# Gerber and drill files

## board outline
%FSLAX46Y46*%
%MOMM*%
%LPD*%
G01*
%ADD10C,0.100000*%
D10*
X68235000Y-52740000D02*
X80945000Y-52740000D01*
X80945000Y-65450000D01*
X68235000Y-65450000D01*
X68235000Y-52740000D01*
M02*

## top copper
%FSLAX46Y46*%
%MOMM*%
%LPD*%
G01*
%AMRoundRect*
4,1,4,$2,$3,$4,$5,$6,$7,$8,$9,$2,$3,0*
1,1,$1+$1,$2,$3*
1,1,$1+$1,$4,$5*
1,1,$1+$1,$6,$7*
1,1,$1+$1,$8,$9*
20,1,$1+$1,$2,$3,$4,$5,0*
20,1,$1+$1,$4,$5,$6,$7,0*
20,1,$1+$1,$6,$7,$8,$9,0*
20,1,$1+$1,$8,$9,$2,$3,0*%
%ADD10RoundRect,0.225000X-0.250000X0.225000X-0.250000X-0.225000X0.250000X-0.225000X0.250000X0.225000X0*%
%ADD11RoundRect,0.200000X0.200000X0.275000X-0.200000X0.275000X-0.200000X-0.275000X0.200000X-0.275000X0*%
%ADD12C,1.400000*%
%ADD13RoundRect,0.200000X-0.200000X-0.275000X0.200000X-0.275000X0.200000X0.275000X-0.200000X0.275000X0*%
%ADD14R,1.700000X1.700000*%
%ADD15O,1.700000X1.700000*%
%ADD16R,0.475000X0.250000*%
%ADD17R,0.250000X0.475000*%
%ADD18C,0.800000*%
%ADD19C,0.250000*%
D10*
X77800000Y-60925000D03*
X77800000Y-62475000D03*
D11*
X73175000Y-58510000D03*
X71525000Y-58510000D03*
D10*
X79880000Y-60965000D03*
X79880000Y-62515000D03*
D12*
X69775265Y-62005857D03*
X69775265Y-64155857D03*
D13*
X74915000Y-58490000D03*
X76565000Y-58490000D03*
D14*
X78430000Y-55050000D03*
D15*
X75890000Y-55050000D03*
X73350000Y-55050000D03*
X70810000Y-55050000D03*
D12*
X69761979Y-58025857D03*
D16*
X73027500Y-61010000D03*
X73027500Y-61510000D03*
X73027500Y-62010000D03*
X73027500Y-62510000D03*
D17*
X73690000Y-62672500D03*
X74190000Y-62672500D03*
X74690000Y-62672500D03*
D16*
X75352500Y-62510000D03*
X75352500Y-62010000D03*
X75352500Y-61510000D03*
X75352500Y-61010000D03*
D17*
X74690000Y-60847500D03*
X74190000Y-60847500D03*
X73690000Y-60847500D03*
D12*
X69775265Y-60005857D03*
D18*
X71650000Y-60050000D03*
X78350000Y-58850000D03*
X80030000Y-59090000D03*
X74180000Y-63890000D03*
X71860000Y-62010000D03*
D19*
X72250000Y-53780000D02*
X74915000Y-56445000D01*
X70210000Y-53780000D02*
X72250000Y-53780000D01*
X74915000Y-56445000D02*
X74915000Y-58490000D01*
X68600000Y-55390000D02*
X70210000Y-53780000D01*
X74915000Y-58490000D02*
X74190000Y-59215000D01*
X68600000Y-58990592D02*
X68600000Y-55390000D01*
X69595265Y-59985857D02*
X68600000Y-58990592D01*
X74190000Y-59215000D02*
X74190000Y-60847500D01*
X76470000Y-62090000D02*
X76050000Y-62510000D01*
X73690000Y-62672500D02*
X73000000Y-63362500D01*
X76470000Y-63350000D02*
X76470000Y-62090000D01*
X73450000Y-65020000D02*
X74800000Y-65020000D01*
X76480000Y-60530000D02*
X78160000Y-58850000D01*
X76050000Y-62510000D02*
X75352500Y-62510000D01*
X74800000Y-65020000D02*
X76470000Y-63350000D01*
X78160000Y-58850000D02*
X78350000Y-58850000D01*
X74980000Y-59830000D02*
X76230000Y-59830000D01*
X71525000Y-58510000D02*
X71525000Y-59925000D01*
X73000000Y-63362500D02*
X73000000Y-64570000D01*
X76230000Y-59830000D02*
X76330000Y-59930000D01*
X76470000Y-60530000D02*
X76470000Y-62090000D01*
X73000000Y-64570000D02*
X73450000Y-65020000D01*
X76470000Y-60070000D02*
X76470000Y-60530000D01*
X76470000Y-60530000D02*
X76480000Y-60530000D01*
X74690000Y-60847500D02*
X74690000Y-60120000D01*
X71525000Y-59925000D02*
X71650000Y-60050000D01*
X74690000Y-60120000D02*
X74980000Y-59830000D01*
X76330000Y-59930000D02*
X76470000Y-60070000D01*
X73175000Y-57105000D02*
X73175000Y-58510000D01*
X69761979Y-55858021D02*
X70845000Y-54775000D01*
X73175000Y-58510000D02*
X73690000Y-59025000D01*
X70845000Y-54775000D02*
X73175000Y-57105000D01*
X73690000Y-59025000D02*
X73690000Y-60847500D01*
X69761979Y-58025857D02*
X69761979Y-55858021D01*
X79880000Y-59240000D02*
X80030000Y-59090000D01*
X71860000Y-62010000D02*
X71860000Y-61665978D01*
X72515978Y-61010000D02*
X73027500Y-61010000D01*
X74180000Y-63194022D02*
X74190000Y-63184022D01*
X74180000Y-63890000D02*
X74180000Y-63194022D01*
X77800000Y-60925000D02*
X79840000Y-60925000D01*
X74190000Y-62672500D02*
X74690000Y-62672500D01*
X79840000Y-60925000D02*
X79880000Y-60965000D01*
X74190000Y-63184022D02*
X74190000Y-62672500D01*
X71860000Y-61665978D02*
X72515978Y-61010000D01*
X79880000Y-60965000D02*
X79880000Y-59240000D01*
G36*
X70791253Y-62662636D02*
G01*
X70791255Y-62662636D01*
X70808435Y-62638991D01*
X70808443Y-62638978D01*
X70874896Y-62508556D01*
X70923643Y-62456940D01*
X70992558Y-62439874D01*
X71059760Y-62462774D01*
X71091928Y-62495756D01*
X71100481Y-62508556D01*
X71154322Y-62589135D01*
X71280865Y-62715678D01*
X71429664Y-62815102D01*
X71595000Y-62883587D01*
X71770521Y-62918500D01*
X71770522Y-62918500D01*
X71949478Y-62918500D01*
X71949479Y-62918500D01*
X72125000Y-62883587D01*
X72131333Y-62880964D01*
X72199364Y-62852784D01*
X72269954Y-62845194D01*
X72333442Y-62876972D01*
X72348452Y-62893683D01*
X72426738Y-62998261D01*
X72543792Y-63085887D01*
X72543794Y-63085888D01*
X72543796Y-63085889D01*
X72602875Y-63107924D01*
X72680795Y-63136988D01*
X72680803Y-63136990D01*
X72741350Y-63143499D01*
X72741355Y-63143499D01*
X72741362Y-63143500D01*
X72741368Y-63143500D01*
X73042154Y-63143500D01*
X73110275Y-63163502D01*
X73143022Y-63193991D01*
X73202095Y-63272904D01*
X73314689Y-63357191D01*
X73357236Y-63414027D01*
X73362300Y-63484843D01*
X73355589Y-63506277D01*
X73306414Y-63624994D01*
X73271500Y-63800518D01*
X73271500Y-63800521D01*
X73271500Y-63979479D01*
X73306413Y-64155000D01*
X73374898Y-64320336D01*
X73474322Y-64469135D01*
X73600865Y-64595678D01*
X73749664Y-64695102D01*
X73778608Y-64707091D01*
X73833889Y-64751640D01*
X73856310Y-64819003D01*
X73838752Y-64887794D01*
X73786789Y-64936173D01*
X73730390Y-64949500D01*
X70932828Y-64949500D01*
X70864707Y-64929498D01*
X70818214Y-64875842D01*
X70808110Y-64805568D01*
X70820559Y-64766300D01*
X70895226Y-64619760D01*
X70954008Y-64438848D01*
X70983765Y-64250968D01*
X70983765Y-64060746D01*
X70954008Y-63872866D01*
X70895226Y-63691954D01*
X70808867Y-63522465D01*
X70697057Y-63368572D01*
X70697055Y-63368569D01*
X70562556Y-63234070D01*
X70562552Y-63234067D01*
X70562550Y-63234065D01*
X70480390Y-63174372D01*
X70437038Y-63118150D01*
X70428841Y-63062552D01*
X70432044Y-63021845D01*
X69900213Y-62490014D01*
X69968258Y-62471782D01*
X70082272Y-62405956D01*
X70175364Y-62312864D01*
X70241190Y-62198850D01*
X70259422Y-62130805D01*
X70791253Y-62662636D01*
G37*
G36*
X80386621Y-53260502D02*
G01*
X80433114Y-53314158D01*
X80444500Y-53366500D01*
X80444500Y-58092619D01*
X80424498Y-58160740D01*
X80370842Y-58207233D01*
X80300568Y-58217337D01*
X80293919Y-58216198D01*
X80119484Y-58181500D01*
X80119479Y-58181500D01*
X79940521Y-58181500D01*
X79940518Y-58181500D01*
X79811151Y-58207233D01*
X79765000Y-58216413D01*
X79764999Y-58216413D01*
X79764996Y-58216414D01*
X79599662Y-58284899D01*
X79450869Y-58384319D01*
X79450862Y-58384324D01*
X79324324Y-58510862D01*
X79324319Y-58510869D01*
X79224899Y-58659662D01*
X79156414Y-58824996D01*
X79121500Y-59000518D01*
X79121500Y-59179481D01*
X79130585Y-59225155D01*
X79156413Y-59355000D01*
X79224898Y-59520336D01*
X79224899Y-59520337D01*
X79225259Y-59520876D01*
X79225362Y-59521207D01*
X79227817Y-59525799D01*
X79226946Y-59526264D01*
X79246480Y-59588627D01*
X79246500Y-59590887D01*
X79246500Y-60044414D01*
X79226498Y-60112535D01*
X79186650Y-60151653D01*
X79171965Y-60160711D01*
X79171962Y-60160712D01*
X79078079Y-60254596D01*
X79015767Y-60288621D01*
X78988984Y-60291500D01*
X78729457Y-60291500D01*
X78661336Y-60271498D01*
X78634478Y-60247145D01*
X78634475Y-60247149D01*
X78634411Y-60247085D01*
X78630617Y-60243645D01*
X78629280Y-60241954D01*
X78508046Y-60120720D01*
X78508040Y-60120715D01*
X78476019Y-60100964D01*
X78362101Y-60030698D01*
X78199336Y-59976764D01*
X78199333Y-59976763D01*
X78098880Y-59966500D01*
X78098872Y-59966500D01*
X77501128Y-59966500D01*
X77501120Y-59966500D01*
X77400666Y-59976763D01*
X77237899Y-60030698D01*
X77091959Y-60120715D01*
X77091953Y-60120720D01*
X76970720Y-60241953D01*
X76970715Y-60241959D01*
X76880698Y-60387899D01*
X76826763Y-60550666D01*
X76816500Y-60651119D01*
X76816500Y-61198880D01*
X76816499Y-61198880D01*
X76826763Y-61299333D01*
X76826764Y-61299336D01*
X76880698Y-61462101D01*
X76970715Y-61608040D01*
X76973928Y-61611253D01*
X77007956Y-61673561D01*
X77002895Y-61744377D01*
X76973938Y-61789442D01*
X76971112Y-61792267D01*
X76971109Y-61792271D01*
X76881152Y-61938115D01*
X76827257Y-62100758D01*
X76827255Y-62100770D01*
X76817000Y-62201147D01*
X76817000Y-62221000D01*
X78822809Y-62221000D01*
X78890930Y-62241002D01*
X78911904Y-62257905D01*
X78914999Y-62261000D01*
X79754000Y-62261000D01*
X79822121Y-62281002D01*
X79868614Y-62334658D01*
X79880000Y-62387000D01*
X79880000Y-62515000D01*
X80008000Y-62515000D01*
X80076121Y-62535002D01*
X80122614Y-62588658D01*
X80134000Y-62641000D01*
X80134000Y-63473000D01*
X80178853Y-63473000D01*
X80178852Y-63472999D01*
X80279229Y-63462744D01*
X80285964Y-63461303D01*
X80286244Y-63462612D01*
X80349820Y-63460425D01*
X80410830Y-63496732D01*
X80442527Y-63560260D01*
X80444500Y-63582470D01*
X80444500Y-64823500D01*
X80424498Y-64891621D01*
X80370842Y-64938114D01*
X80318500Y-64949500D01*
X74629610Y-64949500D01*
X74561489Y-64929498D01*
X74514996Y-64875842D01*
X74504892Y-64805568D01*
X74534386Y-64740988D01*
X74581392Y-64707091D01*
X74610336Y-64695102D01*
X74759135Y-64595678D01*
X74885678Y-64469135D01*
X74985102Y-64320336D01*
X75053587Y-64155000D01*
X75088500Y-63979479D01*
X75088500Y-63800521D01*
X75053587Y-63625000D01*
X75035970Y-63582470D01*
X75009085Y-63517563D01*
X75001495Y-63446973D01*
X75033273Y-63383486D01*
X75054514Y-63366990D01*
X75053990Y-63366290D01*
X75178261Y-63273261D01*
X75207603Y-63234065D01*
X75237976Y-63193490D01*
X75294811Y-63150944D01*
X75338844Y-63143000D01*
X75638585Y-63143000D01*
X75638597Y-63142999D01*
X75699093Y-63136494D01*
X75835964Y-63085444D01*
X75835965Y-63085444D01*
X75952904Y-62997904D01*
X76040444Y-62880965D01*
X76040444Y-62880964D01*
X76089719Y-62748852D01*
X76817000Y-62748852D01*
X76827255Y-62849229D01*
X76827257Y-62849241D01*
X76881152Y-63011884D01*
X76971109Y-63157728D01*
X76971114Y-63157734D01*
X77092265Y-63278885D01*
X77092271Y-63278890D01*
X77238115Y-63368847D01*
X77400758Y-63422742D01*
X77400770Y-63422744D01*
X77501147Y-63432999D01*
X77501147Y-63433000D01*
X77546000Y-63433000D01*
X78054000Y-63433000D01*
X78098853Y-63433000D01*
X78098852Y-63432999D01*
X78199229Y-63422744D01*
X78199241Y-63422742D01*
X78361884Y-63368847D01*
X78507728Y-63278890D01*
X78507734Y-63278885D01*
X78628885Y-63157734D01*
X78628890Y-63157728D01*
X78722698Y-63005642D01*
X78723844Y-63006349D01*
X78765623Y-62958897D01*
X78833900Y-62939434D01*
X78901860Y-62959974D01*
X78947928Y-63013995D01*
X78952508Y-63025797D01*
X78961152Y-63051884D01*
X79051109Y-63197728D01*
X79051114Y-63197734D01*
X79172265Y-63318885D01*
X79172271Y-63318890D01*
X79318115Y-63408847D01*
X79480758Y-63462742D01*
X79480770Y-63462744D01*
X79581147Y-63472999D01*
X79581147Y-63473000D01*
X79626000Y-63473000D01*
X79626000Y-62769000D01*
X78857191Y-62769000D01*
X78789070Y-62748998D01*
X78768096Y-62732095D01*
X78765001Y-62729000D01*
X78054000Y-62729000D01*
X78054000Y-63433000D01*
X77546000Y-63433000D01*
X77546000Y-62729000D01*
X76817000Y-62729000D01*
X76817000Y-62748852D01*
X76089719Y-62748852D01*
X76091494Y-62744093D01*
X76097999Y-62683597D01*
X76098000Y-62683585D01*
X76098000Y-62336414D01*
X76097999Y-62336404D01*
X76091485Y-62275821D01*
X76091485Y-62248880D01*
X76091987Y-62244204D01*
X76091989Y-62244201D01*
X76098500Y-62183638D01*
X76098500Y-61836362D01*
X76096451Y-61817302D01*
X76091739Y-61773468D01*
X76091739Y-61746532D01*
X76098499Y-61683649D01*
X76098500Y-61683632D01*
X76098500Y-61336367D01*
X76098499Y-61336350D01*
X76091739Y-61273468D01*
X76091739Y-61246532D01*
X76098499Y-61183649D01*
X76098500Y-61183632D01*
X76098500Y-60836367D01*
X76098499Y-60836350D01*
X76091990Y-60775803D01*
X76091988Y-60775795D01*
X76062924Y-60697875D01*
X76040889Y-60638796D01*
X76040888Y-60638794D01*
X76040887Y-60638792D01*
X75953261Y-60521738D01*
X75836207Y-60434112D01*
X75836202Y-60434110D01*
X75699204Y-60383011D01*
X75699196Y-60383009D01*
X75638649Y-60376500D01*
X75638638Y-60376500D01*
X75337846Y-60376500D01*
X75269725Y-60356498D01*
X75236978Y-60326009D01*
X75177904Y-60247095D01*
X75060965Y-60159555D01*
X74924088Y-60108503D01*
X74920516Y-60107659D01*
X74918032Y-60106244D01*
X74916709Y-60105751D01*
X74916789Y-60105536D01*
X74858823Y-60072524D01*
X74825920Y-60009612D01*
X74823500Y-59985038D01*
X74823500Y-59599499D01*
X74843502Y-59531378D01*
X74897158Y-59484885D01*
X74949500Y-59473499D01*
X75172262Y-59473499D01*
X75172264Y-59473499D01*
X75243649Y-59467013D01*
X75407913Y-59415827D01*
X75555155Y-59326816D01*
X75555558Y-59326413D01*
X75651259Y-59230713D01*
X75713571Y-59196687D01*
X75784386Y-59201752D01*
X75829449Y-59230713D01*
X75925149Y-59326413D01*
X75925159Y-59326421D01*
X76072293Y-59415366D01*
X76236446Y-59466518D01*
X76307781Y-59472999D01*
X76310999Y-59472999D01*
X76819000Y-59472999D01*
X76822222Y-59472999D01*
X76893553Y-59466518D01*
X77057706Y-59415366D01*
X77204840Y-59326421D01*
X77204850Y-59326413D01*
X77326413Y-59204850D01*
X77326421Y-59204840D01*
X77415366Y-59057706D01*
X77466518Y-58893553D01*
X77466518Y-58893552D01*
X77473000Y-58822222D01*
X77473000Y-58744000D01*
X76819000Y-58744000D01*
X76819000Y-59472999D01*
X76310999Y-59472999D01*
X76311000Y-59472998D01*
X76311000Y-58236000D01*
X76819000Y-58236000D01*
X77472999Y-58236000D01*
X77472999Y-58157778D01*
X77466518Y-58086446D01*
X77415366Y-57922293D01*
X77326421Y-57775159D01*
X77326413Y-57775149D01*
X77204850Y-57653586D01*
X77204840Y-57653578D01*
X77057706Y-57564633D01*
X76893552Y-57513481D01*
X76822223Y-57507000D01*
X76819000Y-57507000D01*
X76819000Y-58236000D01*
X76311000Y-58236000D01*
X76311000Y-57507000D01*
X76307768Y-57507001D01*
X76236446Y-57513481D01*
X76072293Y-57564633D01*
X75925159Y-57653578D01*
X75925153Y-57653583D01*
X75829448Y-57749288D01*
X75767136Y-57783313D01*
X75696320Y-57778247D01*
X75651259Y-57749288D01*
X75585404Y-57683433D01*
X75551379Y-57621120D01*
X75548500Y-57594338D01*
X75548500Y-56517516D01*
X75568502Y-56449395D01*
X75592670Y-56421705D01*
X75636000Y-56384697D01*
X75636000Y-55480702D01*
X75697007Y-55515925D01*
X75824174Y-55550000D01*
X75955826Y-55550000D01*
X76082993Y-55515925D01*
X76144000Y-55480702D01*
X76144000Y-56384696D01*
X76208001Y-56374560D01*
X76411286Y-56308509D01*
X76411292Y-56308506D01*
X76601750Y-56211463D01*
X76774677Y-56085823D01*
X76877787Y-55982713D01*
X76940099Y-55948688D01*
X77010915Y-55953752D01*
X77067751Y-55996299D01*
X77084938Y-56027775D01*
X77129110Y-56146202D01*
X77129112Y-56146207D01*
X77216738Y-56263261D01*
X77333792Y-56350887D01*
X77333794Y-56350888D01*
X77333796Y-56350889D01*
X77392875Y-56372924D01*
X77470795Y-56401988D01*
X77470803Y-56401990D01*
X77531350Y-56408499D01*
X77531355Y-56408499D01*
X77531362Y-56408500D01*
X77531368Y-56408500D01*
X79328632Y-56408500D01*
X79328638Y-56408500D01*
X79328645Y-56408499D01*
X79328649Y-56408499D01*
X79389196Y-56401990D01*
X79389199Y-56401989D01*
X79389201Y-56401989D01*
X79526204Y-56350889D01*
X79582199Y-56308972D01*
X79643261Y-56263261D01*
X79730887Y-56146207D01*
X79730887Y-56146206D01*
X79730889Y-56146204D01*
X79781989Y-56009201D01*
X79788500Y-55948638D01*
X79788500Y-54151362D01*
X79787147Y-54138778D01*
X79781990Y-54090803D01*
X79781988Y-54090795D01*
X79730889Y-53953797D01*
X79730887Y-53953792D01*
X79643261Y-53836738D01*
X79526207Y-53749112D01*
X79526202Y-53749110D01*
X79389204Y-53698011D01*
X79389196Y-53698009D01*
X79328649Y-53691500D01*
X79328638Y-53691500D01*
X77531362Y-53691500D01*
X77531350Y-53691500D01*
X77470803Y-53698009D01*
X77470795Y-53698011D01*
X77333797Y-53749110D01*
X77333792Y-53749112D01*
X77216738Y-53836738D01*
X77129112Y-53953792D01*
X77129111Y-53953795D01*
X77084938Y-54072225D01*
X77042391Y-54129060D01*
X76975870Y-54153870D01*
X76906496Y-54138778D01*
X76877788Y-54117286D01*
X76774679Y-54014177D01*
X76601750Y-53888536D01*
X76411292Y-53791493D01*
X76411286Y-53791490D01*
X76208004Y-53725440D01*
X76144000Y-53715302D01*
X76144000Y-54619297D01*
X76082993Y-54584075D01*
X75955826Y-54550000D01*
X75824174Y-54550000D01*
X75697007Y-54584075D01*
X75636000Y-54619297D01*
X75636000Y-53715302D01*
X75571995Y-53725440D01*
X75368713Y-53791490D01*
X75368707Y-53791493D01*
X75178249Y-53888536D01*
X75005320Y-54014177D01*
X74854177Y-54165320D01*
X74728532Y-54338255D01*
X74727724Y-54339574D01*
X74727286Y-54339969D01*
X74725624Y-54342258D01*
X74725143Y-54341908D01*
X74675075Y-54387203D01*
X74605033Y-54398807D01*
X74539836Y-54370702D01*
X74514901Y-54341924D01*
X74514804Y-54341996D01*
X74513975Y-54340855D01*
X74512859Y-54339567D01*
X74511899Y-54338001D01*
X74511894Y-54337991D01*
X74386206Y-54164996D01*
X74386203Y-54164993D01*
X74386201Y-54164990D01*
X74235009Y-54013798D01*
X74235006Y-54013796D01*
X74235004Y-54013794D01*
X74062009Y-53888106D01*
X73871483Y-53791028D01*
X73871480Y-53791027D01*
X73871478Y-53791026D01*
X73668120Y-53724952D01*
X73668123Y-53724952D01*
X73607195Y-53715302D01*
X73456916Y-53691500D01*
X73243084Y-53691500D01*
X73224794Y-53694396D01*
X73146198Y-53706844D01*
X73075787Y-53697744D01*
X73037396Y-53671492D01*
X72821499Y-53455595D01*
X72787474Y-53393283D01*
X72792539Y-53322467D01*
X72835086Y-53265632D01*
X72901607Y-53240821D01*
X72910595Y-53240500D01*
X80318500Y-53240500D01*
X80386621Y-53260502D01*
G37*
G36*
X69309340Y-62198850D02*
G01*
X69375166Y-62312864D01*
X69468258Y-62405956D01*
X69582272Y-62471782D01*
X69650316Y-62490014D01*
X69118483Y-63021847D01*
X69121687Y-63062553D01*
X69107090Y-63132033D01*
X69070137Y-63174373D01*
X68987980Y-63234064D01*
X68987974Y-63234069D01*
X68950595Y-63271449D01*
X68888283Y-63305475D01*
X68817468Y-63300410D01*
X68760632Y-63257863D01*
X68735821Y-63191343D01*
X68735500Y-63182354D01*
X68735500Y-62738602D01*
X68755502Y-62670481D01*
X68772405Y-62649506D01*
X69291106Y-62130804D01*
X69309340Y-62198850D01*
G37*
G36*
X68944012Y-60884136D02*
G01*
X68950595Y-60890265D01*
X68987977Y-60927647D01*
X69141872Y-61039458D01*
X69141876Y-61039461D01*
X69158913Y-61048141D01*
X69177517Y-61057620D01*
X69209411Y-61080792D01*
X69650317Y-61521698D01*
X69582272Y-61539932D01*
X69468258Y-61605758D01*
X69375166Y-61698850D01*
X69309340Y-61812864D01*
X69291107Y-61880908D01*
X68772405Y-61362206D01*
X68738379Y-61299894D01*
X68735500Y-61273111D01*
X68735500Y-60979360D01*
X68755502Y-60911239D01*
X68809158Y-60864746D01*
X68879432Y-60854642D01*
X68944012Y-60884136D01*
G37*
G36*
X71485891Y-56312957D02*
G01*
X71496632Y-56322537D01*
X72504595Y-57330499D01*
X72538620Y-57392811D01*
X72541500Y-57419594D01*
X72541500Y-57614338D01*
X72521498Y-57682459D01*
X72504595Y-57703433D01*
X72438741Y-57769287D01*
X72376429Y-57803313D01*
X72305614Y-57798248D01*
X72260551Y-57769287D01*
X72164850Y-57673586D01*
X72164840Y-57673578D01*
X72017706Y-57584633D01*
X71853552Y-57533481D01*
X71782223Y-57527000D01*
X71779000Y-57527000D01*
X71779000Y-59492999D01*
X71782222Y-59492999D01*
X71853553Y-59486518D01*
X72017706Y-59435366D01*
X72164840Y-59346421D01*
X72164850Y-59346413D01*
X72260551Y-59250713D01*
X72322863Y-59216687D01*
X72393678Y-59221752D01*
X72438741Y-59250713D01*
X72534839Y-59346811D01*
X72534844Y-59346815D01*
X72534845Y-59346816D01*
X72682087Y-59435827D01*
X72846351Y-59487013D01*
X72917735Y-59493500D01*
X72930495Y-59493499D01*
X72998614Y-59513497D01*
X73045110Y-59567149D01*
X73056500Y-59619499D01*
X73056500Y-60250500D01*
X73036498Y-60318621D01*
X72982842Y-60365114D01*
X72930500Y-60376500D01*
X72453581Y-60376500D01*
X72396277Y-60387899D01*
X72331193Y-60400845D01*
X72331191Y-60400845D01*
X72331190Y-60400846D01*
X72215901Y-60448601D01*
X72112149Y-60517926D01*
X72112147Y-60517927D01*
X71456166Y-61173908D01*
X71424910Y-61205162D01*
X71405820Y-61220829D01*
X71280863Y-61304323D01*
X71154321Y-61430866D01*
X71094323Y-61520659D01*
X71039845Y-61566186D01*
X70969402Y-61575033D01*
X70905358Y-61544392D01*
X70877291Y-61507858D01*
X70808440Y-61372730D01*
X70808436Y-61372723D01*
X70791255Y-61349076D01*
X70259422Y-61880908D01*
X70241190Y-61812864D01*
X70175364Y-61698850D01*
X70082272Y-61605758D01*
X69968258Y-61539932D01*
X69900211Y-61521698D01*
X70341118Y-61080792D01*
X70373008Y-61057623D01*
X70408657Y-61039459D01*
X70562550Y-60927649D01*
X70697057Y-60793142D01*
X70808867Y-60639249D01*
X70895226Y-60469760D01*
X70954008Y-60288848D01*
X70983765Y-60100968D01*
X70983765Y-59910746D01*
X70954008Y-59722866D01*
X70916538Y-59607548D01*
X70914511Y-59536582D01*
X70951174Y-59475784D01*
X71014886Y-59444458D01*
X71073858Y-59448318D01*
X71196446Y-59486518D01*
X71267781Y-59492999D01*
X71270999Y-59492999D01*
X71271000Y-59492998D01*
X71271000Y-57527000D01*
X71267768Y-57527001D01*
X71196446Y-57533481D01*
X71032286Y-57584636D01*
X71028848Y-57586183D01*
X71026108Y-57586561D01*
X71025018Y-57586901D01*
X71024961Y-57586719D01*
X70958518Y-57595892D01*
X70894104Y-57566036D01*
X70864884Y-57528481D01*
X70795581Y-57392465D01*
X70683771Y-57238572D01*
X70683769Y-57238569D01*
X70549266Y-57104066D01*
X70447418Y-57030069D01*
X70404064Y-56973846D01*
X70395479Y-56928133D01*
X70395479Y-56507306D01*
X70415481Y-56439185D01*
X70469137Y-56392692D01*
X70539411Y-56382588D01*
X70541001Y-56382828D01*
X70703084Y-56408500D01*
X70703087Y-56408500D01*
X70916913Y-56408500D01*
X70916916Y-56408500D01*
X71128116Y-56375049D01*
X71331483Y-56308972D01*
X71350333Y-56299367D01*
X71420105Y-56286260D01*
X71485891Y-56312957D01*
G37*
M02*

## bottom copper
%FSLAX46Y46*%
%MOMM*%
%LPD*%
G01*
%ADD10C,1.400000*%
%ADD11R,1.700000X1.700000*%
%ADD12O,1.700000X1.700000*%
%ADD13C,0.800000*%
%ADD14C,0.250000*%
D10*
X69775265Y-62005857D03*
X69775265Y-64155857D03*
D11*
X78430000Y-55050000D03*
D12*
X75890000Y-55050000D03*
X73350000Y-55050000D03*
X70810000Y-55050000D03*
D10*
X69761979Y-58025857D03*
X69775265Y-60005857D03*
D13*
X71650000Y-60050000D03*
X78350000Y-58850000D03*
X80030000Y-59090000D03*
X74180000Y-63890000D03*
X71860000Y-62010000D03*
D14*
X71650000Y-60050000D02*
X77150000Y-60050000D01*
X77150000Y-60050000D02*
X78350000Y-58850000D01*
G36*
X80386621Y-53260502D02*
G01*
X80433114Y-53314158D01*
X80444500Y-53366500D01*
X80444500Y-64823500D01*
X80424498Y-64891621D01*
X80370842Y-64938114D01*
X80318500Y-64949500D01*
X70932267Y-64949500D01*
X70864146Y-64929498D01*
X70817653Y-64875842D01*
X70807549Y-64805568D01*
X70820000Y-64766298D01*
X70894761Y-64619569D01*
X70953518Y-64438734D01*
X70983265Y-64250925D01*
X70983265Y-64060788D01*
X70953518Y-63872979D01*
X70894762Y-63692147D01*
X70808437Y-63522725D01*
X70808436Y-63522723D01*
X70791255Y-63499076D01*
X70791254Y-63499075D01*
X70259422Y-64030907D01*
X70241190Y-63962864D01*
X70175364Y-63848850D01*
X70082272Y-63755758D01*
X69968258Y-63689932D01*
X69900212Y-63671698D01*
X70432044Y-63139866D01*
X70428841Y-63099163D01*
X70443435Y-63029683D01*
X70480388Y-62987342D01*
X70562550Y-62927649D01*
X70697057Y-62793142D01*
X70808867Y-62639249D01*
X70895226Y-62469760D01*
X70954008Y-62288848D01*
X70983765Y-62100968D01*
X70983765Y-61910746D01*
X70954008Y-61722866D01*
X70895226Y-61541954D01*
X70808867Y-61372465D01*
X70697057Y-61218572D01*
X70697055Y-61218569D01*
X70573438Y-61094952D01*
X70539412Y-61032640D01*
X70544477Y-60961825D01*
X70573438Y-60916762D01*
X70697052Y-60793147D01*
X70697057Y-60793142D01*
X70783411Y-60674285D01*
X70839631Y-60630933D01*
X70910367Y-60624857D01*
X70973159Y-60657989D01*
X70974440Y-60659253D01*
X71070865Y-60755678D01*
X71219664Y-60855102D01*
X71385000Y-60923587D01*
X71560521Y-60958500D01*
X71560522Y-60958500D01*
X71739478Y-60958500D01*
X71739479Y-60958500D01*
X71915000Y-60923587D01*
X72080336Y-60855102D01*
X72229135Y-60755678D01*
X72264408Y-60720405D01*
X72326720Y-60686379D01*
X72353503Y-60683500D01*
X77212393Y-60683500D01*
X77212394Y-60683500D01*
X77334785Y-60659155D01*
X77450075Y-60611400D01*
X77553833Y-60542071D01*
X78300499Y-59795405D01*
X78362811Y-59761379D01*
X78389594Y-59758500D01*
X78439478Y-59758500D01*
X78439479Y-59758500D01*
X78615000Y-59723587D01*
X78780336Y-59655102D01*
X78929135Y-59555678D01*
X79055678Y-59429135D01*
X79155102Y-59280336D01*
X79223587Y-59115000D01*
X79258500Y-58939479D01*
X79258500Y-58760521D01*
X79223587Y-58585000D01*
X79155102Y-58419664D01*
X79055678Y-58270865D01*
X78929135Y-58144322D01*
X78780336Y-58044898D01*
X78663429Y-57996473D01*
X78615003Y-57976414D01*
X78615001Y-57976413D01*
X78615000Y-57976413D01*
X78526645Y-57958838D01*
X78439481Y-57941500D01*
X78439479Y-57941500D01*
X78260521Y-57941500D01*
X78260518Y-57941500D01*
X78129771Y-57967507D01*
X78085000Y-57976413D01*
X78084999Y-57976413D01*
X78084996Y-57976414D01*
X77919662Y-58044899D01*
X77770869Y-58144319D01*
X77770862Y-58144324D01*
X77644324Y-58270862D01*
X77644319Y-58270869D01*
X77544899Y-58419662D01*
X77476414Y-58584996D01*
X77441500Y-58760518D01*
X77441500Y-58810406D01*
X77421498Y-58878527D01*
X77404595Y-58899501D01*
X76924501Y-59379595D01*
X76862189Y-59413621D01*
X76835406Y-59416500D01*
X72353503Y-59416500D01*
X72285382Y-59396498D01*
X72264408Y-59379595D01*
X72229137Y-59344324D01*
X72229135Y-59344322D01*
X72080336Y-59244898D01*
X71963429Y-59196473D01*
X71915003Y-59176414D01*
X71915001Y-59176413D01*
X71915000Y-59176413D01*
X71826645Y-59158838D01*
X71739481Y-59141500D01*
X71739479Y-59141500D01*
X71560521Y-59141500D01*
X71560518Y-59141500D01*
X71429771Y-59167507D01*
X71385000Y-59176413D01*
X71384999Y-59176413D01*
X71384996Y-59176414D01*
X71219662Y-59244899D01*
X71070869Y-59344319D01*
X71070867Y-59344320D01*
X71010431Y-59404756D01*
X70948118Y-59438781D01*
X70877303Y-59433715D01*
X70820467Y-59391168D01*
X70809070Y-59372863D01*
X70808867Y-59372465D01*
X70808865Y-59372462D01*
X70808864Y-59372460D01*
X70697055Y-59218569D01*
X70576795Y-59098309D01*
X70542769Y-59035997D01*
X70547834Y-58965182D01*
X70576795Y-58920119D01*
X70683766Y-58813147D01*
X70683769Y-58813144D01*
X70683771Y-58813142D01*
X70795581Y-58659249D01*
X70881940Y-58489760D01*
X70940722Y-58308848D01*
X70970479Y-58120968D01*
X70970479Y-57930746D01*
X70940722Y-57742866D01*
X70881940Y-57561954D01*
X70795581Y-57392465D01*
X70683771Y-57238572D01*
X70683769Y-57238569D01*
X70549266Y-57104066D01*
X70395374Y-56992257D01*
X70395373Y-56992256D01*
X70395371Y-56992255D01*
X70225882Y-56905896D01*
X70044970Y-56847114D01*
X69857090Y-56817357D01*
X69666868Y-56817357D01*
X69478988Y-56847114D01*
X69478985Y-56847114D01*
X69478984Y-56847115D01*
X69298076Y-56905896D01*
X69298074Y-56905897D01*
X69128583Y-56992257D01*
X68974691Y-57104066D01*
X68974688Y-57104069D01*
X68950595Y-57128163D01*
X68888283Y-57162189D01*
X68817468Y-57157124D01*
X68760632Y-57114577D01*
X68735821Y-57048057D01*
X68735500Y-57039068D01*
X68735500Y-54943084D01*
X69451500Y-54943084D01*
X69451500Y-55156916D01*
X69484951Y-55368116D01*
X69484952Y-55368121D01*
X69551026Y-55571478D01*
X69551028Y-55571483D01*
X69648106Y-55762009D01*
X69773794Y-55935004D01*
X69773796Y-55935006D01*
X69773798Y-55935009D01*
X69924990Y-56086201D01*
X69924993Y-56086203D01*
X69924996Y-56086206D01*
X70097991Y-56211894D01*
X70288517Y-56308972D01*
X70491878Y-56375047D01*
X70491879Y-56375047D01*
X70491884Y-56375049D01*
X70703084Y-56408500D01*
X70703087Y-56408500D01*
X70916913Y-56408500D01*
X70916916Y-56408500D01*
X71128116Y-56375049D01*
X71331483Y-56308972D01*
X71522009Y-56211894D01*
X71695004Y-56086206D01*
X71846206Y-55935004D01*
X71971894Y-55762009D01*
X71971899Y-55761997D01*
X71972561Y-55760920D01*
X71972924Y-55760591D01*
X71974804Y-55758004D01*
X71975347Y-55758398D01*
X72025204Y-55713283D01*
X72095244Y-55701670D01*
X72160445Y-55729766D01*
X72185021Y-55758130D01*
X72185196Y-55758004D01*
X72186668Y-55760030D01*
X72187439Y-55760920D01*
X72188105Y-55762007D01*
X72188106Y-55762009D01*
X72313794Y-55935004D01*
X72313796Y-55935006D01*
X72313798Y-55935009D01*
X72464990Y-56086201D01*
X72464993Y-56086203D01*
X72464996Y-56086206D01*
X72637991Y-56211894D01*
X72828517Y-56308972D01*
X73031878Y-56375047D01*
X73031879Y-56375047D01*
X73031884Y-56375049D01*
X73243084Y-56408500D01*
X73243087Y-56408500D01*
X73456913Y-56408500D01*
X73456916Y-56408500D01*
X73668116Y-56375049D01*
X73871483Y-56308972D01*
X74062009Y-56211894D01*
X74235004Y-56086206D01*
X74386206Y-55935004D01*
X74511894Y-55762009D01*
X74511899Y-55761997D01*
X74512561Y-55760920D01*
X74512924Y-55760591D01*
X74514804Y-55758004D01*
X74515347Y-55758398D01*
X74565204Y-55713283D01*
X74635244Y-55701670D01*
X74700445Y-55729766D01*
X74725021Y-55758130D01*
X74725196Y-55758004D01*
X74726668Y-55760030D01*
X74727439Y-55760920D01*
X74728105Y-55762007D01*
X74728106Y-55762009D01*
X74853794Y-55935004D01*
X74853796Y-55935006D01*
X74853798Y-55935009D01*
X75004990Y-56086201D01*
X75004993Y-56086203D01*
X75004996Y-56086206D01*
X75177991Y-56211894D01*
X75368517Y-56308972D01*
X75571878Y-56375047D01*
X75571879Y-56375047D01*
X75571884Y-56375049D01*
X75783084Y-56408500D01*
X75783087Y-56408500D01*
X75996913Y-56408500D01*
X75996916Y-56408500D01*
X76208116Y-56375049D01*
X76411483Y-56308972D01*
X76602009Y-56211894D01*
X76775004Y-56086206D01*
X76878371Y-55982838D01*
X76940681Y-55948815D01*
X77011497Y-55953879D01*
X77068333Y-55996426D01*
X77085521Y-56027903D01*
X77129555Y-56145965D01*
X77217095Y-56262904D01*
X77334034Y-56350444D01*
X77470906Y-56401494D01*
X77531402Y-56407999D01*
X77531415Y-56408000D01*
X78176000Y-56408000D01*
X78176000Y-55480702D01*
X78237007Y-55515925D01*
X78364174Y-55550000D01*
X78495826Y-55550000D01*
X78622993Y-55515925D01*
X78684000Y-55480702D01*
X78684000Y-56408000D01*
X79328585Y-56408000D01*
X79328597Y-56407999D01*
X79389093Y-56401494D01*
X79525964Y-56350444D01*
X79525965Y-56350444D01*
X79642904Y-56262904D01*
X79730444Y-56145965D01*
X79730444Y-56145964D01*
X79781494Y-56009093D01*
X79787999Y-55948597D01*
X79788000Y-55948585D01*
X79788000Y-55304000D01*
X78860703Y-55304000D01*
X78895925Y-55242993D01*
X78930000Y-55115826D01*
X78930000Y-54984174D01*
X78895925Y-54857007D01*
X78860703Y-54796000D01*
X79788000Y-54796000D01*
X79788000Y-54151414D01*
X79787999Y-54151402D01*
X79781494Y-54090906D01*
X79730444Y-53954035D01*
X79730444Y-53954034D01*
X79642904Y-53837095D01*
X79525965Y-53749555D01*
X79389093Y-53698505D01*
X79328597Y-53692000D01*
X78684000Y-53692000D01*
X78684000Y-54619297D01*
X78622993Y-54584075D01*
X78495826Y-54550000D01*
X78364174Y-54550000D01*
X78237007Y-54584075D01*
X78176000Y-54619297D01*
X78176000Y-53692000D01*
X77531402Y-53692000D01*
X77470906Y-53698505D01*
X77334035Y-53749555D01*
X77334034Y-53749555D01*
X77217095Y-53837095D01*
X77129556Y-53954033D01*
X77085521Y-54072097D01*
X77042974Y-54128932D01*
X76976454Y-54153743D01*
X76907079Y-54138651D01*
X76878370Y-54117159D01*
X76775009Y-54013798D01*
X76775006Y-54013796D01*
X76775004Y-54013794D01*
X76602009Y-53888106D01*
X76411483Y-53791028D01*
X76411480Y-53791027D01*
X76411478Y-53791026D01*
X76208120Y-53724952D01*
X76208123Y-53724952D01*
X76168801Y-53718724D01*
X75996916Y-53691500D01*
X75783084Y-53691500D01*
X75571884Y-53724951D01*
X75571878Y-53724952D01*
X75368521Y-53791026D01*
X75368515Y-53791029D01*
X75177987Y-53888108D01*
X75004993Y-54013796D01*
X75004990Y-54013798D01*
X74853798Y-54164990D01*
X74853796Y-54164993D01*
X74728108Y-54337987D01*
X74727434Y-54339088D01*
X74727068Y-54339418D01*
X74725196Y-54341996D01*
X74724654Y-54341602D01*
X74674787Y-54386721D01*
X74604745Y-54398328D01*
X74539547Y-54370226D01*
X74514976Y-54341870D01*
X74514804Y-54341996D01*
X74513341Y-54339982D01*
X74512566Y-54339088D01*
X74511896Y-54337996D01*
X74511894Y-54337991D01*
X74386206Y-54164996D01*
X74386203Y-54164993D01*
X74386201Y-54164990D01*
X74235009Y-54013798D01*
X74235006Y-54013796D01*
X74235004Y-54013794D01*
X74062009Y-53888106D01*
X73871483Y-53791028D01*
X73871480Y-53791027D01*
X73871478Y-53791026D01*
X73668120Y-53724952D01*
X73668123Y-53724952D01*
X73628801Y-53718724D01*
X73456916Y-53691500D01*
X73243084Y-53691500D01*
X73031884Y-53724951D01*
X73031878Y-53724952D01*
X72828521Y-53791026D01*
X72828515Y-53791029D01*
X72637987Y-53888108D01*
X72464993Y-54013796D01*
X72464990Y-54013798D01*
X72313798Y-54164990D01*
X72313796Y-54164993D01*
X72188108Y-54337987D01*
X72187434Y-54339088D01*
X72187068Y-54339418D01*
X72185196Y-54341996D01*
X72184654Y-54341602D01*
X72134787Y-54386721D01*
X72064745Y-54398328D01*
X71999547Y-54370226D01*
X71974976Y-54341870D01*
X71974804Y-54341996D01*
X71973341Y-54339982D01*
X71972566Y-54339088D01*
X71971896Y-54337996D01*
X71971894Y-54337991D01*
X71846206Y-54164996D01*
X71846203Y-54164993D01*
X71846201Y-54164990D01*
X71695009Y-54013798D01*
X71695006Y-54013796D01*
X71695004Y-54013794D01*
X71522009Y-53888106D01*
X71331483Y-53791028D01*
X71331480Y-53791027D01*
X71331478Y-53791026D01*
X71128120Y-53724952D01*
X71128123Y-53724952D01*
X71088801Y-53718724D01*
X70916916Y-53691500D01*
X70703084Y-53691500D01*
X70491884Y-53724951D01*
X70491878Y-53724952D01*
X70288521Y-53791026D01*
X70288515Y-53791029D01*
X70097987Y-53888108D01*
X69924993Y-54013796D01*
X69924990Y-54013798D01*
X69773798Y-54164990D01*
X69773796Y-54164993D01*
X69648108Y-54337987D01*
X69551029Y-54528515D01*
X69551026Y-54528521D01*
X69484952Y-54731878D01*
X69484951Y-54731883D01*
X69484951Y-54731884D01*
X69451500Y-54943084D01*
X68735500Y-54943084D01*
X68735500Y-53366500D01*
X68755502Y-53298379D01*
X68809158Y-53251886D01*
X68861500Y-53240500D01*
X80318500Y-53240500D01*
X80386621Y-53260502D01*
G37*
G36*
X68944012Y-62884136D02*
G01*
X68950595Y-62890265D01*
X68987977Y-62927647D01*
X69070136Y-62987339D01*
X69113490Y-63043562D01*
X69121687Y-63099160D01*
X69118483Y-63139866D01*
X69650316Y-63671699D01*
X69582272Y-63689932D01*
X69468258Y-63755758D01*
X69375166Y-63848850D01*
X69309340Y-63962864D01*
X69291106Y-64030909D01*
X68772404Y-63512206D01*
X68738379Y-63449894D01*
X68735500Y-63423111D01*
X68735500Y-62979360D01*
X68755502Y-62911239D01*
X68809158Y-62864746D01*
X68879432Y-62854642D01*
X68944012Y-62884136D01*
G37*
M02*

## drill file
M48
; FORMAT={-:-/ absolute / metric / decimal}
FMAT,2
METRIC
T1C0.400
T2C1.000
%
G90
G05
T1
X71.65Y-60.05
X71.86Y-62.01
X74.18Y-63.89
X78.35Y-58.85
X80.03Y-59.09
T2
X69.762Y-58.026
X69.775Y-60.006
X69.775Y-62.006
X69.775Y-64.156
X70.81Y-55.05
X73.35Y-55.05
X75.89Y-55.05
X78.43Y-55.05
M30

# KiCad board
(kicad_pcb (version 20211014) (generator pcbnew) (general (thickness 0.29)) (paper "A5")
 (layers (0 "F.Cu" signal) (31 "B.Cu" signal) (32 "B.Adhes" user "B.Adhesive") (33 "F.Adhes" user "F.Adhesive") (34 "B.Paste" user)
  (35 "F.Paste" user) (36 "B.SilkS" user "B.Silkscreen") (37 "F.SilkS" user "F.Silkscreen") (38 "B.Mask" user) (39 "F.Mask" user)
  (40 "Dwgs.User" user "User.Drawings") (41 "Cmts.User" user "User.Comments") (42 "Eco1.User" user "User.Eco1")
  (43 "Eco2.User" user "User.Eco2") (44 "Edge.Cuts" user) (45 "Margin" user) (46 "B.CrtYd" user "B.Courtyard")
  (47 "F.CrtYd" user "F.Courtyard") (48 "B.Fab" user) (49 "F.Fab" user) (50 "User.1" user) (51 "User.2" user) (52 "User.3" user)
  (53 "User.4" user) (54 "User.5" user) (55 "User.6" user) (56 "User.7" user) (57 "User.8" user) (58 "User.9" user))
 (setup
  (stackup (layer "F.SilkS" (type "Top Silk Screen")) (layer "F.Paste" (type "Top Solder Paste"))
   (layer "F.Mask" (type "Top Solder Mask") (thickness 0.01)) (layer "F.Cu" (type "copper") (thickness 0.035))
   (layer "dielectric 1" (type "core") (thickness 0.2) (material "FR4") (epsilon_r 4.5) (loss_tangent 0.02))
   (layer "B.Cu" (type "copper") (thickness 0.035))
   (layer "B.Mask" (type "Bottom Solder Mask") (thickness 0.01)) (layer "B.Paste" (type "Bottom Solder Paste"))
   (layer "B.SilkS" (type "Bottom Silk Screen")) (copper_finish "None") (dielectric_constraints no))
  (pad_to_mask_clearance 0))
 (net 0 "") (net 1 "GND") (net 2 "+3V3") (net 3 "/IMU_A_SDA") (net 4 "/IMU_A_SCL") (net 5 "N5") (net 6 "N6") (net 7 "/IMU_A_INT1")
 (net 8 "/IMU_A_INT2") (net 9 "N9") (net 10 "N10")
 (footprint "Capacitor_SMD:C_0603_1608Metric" (layer "F.Cu") (at 77.8 61.7 -90)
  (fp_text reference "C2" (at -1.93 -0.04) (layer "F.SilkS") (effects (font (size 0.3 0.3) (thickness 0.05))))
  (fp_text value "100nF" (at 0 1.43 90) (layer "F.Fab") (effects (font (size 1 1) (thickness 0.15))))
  (pad "1" smd roundrect (at -0.775 0 270) (size 0.9 0.95) (layers "F.Cu" "F.Paste" "F.Mask") (roundrect_rratio 0.25) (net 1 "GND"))
  (pad "2" smd roundrect (at 0.775 0 270) (size 0.9 0.95) (layers "F.Cu" "F.Paste" "F.Mask") (roundrect_rratio 0.25) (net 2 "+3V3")))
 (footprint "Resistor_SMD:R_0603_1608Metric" (layer "F.Cu") (at 72.35 58.51 180)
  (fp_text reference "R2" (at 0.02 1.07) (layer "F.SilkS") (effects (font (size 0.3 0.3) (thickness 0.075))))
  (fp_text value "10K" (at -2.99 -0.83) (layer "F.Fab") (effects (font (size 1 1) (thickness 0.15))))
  (pad "1" smd roundrect (at -0.825 0 180) (size 0.8 0.95) (layers "F.Cu" "F.Paste" "F.Mask") (roundrect_rratio 0.25) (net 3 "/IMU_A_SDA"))
  (pad "2" smd roundrect (at 0.825 0 180) (size 0.8 0.95) (layers "F.Cu" "F.Paste" "F.Mask") (roundrect_rratio 0.25) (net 2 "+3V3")))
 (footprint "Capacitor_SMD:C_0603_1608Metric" (layer "F.Cu") (at 79.88 61.74 -90)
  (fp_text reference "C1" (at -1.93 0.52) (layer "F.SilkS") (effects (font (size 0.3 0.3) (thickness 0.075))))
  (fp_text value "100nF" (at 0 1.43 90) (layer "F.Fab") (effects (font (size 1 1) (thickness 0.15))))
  (pad "1" smd roundrect (at -0.775 0 270) (size 0.9 0.95) (layers "F.Cu" "F.Paste" "F.Mask") (roundrect_rratio 0.25) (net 1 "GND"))
  (pad "2" smd roundrect (at 0.775 0 270) (size 0.9 0.95) (layers "F.Cu" "F.Paste" "F.Mask") (roundrect_rratio 0.25) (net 2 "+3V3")))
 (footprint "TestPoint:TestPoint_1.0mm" (layer "F.Cu") (at 69.78 62.02 -90)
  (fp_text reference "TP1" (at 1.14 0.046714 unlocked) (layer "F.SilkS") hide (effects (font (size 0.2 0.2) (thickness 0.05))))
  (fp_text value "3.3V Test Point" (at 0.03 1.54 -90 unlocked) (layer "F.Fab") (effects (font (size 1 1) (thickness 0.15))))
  (pad "1" thru_hole circle (at -0.014143 0.004735 270) (size 1.4 1.4) (drill 1) (layers *.Cu *.Mask) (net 2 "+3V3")))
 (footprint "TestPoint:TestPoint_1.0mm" (layer "F.Cu") (at 69.78 64.17 -90)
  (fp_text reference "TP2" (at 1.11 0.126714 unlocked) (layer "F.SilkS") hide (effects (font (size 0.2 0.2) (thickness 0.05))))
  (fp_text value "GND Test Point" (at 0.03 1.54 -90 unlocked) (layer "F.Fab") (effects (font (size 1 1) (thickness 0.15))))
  (pad "1" thru_hole circle (at -0.014143 0.004735 270) (size 1.4 1.4) (drill 1) (layers *.Cu *.Mask) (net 1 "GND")))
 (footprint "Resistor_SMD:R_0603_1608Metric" (layer "F.Cu") (at 75.74 58.49)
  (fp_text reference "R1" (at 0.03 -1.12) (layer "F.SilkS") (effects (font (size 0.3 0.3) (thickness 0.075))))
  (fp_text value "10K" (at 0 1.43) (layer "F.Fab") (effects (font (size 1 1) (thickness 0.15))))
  (pad "1" smd roundrect (at -0.825 0) (size 0.8 0.95) (layers "F.Cu" "F.Paste" "F.Mask") (roundrect_rratio 0.25) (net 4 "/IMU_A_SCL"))
  (pad "2" smd roundrect (at 0.825 0) (size 0.8 0.95) (layers "F.Cu" "F.Paste" "F.Mask") (roundrect_rratio 0.25) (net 2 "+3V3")))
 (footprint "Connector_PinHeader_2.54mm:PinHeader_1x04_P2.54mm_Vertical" (layer "F.Cu") (at 78.43 55.05 -90)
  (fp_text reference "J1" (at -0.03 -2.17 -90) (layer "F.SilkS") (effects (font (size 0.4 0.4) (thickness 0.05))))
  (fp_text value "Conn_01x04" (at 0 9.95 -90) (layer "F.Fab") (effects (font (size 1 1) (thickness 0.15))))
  (pad "1" thru_hole rect (at 0 0 270) (size 1.7 1.7) (drill 1) (layers *.Cu *.Mask) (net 1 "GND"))
  (pad "2" thru_hole oval (at 0 2.54 270) (size 1.7 1.7) (drill 1) (layers *.Cu *.Mask) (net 2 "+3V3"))
  (pad "3" thru_hole oval (at 0 5.08 270) (size 1.7 1.7) (drill 1) (layers *.Cu *.Mask) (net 4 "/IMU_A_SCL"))
  (pad "4" thru_hole oval (at 0 7.62 270) (size 1.7 1.7) (drill 1) (layers *.Cu *.Mask) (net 3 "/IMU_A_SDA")))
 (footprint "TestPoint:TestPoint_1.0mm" (layer "F.Cu") (at 69.766714 58.04 -90)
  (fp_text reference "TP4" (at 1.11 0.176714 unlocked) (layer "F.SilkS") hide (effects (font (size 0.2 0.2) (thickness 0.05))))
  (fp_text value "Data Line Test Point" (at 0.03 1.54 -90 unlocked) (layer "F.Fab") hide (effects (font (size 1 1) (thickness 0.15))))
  (pad "1" thru_hole circle (at -0.014143 0.004735 270) (size 1.4 1.4) (drill 1) (layers *.Cu *.Mask) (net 3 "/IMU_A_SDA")))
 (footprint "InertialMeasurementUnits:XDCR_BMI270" (layer "F.Cu") (at 74.19 61.76)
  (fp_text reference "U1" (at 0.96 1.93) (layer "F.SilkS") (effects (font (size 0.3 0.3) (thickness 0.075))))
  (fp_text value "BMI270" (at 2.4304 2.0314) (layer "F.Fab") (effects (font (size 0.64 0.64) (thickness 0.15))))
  (pad "1" smd rect locked (at -1.1625 -0.75) (size 0.475 0.25) (layers "F.Cu" "F.Paste" "F.Mask") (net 1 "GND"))
  (pad "2" smd rect locked (at -1.1625 -0.25) (size 0.475 0.25) (layers "F.Cu" "F.Paste" "F.Mask") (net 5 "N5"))
  (pad "3" smd rect locked (at -1.1625 0.25) (size 0.475 0.25) (layers "F.Cu" "F.Paste" "F.Mask") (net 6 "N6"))
  (pad "4" smd rect locked (at -1.1625 0.75) (size 0.475 0.25) (layers "F.Cu" "F.Paste" "F.Mask") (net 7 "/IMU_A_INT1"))
  (pad "5" smd rect locked (at -0.5 0.9125) (size 0.25 0.475) (layers "F.Cu" "F.Paste" "F.Mask") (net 2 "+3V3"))
  (pad "6" smd rect locked (at 0 0.9125) (size 0.25 0.475) (layers "F.Cu" "F.Paste" "F.Mask") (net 1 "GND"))
  (pad "7" smd rect locked (at 0.5 0.9125) (size 0.25 0.475) (layers "F.Cu" "F.Paste" "F.Mask") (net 1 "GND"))
  (pad "8" smd rect locked (at 1.1625 0.75) (size 0.475 0.25) (layers "F.Cu" "F.Paste" "F.Mask") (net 2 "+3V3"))
  (pad "9" smd rect locked (at 1.1625 0.25) (size 0.475 0.25) (layers "F.Cu" "F.Paste" "F.Mask") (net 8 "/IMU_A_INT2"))
  (pad "10" smd rect locked (at 1.1625 -0.25) (size 0.475 0.25) (layers "F.Cu" "F.Paste" "F.Mask") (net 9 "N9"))
  (pad "11" smd rect locked (at 1.1625 -0.75) (size 0.475 0.25) (layers "F.Cu" "F.Paste" "F.Mask") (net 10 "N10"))
  (pad "12" smd rect locked (at 0.5 -0.9125) (size 0.25 0.475) (layers "F.Cu" "F.Paste" "F.Mask") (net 2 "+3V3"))
  (pad "13" smd rect locked (at 0 -0.9125) (size 0.25 0.475) (layers "F.Cu" "F.Paste" "F.Mask") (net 4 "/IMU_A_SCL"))
  (pad "14" smd rect locked (at -0.5 -0.9125) (size 0.25 0.475) (layers "F.Cu" "F.Paste" "F.Mask") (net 3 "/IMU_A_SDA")))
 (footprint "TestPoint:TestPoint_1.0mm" (layer "F.Cu") (at 69.78 60.02 -90)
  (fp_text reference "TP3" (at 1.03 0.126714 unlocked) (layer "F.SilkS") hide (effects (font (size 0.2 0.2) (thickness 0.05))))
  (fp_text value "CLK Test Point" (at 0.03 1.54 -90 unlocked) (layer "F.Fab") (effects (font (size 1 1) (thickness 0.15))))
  (pad "1" thru_hole circle (at -0.014143 0.004735 270) (size 1.4 1.4) (drill 1) (layers *.Cu *.Mask) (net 4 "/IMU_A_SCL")))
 (gr_rect (start 68.235 52.74) (end 80.945 65.45) (layer "Edge.Cuts") (width 0.1) (fill none))
 (segment (start 72.25 53.78) (end 74.915 56.445) (width 0.25) (layer "F.Cu") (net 4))
 (segment (start 70.21 53.78) (end 72.25 53.78) (width 0.25) (layer "F.Cu") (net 4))
 (segment (start 74.915 56.445) (end 74.915 58.49) (width 0.25) (layer "F.Cu") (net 4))
 (segment (start 68.6 55.39) (end 70.21 53.78) (width 0.25) (layer "F.Cu") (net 4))
 (segment (start 74.915 58.49) (end 74.19 59.215) (width 0.25) (layer "F.Cu") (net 4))
 (segment (start 68.6 58.990592) (end 68.6 55.39) (width 0.25) (layer "F.Cu") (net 4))
 (segment (start 69.595265 59.985857) (end 68.6 58.990592) (width 0.25) (layer "F.Cu") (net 4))
 (segment (start 74.19 59.215) (end 74.19 60.8475) (width 0.25) (layer "F.Cu") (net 4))
 (segment (start 76.47 62.09) (end 76.05 62.51) (width 0.25) (layer "F.Cu") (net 2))
 (segment (start 73.69 62.6725) (end 73 63.3625) (width 0.25) (layer "F.Cu") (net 2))
 (segment (start 76.47 63.35) (end 76.47 62.09) (width 0.25) (layer "F.Cu") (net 2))
 (segment (start 73.45 65.02) (end 74.8 65.02) (width 0.25) (layer "F.Cu") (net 2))
 (segment (start 76.48 60.53) (end 78.16 58.85) (width 0.25) (layer "F.Cu") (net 2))
 (segment (start 76.05 62.51) (end 75.3525 62.51) (width 0.25) (layer "F.Cu") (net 2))
 (segment (start 74.8 65.02) (end 76.47 63.35) (width 0.25) (layer "F.Cu") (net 2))
 (segment (start 78.16 58.85) (end 78.35 58.85) (width 0.25) (layer "F.Cu") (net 2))
 (segment (start 74.98 59.83) (end 76.23 59.83) (width 0.25) (layer "F.Cu") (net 2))
 (segment (start 71.525 58.51) (end 71.525 59.925) (width 0.25) (layer "F.Cu") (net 2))
 (segment (start 73 63.3625) (end 73 64.57) (width 0.25) (layer "F.Cu") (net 2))
 (segment (start 76.23 59.83) (end 76.33 59.93) (width 0.25) (layer "F.Cu") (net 2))
 (segment (start 76.47 60.53) (end 76.47 62.09) (width 0.25) (layer "F.Cu") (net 2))
 (segment (start 73 64.57) (end 73.45 65.02) (width 0.25) (layer "F.Cu") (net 2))
 (segment (start 76.47 60.07) (end 76.47 60.53) (width 0.25) (layer "F.Cu") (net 2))
 (segment (start 76.47 60.53) (end 76.48 60.53) (width 0.25) (layer "F.Cu") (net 2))
 (segment (start 74.69 60.8475) (end 74.69 60.12) (width 0.25) (layer "F.Cu") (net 2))
 (segment (start 71.525 59.925) (end 71.65 60.05) (width 0.25) (layer "F.Cu") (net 2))
 (segment (start 74.69 60.12) (end 74.98 59.83) (width 0.25) (layer "F.Cu") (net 2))
 (segment (start 76.33 59.93) (end 76.47 60.07) (width 0.25) (layer "F.Cu") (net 2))
 (via (at 71.65 60.05) (size 0.8) (drill 0.4) (layers "F.Cu" "B.Cu") (free) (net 2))
 (via (at 78.35 58.85) (size 0.8) (drill 0.4) (layers "F.Cu" "B.Cu") (free) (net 2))
 (segment (start 71.65 60.05) (end 77.15 60.05) (width 0.25) (layer "B.Cu") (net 2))
 (segment (start 77.15 60.05) (end 78.35 58.85) (width 0.25) (layer "B.Cu") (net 2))
 (segment (start 73.175 57.105) (end 73.175 58.51) (width 0.25) (layer "F.Cu") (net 3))
 (segment (start 69.761979 55.858021) (end 70.845 54.775) (width 0.25) (layer "F.Cu") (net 3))
 (segment (start 73.175 58.51) (end 73.69 59.025) (width 0.25) (layer "F.Cu") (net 3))
 (segment (start 70.845 54.775) (end 73.175 57.105) (width 0.25) (layer "F.Cu") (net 3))
 (segment (start 73.69 59.025) (end 73.69 60.8475) (width 0.25) (layer "F.Cu") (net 3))
 (segment (start 69.761979 58.025857) (end 69.761979 55.858021) (width 0.25) (layer "F.Cu") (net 3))
 (segment (start 79.88 59.24) (end 80.03 59.09) (width 0.25) (layer "F.Cu") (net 1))
 (segment (start 71.86 62.01) (end 71.86 61.665978) (width 0.25) (layer "F.Cu") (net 1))
 (segment (start 72.515978 61.01) (end 73.0275 61.01) (width 0.25) (layer "F.Cu") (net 1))
 (segment (start 74.18 63.194022) (end 74.19 63.184022) (width 0.25) (layer "F.Cu") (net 1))
 (segment (start 74.18 63.89) (end 74.18 63.194022) (width 0.25) (layer "F.Cu") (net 1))
 (segment (start 77.8 60.925) (end 79.84 60.925) (width 0.25) (layer "F.Cu") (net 1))
 (segment (start 74.19 62.6725) (end 74.69 62.6725) (width 0.25) (layer "F.Cu") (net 1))
 (segment (start 79.84 60.925) (end 79.88 60.965) (width 0.25) (layer "F.Cu") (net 1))
 (segment (start 74.19 63.184022) (end 74.19 62.6725) (width 0.25) (layer "F.Cu") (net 1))
 (segment (start 71.86 61.665978) (end 72.515978 61.01) (width 0.25) (layer "F.Cu") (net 1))
 (segment (start 79.88 60.965) (end 79.88 59.24) (width 0.25) (layer "F.Cu") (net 1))
 (via (at 80.03 59.09) (size 0.8) (drill 0.4) (layers "F.Cu" "B.Cu") (free) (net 1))
 (via (at 74.18 63.89) (size 0.8) (drill 0.4) (layers "F.Cu" "B.Cu") (free) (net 1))
 (via (at 71.86 62.01) (size 0.8) (drill 0.4) (layers "F.Cu" "B.Cu") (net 1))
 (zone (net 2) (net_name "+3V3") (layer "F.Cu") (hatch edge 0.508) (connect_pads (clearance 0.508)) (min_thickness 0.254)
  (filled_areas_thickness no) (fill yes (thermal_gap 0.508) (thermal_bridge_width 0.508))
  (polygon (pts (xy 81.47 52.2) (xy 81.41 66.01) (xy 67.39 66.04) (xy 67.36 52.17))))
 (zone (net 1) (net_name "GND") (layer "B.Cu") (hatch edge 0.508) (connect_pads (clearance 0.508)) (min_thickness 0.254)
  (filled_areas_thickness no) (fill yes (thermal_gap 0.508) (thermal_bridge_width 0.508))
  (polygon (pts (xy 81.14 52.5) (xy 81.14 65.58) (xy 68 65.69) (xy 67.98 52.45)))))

